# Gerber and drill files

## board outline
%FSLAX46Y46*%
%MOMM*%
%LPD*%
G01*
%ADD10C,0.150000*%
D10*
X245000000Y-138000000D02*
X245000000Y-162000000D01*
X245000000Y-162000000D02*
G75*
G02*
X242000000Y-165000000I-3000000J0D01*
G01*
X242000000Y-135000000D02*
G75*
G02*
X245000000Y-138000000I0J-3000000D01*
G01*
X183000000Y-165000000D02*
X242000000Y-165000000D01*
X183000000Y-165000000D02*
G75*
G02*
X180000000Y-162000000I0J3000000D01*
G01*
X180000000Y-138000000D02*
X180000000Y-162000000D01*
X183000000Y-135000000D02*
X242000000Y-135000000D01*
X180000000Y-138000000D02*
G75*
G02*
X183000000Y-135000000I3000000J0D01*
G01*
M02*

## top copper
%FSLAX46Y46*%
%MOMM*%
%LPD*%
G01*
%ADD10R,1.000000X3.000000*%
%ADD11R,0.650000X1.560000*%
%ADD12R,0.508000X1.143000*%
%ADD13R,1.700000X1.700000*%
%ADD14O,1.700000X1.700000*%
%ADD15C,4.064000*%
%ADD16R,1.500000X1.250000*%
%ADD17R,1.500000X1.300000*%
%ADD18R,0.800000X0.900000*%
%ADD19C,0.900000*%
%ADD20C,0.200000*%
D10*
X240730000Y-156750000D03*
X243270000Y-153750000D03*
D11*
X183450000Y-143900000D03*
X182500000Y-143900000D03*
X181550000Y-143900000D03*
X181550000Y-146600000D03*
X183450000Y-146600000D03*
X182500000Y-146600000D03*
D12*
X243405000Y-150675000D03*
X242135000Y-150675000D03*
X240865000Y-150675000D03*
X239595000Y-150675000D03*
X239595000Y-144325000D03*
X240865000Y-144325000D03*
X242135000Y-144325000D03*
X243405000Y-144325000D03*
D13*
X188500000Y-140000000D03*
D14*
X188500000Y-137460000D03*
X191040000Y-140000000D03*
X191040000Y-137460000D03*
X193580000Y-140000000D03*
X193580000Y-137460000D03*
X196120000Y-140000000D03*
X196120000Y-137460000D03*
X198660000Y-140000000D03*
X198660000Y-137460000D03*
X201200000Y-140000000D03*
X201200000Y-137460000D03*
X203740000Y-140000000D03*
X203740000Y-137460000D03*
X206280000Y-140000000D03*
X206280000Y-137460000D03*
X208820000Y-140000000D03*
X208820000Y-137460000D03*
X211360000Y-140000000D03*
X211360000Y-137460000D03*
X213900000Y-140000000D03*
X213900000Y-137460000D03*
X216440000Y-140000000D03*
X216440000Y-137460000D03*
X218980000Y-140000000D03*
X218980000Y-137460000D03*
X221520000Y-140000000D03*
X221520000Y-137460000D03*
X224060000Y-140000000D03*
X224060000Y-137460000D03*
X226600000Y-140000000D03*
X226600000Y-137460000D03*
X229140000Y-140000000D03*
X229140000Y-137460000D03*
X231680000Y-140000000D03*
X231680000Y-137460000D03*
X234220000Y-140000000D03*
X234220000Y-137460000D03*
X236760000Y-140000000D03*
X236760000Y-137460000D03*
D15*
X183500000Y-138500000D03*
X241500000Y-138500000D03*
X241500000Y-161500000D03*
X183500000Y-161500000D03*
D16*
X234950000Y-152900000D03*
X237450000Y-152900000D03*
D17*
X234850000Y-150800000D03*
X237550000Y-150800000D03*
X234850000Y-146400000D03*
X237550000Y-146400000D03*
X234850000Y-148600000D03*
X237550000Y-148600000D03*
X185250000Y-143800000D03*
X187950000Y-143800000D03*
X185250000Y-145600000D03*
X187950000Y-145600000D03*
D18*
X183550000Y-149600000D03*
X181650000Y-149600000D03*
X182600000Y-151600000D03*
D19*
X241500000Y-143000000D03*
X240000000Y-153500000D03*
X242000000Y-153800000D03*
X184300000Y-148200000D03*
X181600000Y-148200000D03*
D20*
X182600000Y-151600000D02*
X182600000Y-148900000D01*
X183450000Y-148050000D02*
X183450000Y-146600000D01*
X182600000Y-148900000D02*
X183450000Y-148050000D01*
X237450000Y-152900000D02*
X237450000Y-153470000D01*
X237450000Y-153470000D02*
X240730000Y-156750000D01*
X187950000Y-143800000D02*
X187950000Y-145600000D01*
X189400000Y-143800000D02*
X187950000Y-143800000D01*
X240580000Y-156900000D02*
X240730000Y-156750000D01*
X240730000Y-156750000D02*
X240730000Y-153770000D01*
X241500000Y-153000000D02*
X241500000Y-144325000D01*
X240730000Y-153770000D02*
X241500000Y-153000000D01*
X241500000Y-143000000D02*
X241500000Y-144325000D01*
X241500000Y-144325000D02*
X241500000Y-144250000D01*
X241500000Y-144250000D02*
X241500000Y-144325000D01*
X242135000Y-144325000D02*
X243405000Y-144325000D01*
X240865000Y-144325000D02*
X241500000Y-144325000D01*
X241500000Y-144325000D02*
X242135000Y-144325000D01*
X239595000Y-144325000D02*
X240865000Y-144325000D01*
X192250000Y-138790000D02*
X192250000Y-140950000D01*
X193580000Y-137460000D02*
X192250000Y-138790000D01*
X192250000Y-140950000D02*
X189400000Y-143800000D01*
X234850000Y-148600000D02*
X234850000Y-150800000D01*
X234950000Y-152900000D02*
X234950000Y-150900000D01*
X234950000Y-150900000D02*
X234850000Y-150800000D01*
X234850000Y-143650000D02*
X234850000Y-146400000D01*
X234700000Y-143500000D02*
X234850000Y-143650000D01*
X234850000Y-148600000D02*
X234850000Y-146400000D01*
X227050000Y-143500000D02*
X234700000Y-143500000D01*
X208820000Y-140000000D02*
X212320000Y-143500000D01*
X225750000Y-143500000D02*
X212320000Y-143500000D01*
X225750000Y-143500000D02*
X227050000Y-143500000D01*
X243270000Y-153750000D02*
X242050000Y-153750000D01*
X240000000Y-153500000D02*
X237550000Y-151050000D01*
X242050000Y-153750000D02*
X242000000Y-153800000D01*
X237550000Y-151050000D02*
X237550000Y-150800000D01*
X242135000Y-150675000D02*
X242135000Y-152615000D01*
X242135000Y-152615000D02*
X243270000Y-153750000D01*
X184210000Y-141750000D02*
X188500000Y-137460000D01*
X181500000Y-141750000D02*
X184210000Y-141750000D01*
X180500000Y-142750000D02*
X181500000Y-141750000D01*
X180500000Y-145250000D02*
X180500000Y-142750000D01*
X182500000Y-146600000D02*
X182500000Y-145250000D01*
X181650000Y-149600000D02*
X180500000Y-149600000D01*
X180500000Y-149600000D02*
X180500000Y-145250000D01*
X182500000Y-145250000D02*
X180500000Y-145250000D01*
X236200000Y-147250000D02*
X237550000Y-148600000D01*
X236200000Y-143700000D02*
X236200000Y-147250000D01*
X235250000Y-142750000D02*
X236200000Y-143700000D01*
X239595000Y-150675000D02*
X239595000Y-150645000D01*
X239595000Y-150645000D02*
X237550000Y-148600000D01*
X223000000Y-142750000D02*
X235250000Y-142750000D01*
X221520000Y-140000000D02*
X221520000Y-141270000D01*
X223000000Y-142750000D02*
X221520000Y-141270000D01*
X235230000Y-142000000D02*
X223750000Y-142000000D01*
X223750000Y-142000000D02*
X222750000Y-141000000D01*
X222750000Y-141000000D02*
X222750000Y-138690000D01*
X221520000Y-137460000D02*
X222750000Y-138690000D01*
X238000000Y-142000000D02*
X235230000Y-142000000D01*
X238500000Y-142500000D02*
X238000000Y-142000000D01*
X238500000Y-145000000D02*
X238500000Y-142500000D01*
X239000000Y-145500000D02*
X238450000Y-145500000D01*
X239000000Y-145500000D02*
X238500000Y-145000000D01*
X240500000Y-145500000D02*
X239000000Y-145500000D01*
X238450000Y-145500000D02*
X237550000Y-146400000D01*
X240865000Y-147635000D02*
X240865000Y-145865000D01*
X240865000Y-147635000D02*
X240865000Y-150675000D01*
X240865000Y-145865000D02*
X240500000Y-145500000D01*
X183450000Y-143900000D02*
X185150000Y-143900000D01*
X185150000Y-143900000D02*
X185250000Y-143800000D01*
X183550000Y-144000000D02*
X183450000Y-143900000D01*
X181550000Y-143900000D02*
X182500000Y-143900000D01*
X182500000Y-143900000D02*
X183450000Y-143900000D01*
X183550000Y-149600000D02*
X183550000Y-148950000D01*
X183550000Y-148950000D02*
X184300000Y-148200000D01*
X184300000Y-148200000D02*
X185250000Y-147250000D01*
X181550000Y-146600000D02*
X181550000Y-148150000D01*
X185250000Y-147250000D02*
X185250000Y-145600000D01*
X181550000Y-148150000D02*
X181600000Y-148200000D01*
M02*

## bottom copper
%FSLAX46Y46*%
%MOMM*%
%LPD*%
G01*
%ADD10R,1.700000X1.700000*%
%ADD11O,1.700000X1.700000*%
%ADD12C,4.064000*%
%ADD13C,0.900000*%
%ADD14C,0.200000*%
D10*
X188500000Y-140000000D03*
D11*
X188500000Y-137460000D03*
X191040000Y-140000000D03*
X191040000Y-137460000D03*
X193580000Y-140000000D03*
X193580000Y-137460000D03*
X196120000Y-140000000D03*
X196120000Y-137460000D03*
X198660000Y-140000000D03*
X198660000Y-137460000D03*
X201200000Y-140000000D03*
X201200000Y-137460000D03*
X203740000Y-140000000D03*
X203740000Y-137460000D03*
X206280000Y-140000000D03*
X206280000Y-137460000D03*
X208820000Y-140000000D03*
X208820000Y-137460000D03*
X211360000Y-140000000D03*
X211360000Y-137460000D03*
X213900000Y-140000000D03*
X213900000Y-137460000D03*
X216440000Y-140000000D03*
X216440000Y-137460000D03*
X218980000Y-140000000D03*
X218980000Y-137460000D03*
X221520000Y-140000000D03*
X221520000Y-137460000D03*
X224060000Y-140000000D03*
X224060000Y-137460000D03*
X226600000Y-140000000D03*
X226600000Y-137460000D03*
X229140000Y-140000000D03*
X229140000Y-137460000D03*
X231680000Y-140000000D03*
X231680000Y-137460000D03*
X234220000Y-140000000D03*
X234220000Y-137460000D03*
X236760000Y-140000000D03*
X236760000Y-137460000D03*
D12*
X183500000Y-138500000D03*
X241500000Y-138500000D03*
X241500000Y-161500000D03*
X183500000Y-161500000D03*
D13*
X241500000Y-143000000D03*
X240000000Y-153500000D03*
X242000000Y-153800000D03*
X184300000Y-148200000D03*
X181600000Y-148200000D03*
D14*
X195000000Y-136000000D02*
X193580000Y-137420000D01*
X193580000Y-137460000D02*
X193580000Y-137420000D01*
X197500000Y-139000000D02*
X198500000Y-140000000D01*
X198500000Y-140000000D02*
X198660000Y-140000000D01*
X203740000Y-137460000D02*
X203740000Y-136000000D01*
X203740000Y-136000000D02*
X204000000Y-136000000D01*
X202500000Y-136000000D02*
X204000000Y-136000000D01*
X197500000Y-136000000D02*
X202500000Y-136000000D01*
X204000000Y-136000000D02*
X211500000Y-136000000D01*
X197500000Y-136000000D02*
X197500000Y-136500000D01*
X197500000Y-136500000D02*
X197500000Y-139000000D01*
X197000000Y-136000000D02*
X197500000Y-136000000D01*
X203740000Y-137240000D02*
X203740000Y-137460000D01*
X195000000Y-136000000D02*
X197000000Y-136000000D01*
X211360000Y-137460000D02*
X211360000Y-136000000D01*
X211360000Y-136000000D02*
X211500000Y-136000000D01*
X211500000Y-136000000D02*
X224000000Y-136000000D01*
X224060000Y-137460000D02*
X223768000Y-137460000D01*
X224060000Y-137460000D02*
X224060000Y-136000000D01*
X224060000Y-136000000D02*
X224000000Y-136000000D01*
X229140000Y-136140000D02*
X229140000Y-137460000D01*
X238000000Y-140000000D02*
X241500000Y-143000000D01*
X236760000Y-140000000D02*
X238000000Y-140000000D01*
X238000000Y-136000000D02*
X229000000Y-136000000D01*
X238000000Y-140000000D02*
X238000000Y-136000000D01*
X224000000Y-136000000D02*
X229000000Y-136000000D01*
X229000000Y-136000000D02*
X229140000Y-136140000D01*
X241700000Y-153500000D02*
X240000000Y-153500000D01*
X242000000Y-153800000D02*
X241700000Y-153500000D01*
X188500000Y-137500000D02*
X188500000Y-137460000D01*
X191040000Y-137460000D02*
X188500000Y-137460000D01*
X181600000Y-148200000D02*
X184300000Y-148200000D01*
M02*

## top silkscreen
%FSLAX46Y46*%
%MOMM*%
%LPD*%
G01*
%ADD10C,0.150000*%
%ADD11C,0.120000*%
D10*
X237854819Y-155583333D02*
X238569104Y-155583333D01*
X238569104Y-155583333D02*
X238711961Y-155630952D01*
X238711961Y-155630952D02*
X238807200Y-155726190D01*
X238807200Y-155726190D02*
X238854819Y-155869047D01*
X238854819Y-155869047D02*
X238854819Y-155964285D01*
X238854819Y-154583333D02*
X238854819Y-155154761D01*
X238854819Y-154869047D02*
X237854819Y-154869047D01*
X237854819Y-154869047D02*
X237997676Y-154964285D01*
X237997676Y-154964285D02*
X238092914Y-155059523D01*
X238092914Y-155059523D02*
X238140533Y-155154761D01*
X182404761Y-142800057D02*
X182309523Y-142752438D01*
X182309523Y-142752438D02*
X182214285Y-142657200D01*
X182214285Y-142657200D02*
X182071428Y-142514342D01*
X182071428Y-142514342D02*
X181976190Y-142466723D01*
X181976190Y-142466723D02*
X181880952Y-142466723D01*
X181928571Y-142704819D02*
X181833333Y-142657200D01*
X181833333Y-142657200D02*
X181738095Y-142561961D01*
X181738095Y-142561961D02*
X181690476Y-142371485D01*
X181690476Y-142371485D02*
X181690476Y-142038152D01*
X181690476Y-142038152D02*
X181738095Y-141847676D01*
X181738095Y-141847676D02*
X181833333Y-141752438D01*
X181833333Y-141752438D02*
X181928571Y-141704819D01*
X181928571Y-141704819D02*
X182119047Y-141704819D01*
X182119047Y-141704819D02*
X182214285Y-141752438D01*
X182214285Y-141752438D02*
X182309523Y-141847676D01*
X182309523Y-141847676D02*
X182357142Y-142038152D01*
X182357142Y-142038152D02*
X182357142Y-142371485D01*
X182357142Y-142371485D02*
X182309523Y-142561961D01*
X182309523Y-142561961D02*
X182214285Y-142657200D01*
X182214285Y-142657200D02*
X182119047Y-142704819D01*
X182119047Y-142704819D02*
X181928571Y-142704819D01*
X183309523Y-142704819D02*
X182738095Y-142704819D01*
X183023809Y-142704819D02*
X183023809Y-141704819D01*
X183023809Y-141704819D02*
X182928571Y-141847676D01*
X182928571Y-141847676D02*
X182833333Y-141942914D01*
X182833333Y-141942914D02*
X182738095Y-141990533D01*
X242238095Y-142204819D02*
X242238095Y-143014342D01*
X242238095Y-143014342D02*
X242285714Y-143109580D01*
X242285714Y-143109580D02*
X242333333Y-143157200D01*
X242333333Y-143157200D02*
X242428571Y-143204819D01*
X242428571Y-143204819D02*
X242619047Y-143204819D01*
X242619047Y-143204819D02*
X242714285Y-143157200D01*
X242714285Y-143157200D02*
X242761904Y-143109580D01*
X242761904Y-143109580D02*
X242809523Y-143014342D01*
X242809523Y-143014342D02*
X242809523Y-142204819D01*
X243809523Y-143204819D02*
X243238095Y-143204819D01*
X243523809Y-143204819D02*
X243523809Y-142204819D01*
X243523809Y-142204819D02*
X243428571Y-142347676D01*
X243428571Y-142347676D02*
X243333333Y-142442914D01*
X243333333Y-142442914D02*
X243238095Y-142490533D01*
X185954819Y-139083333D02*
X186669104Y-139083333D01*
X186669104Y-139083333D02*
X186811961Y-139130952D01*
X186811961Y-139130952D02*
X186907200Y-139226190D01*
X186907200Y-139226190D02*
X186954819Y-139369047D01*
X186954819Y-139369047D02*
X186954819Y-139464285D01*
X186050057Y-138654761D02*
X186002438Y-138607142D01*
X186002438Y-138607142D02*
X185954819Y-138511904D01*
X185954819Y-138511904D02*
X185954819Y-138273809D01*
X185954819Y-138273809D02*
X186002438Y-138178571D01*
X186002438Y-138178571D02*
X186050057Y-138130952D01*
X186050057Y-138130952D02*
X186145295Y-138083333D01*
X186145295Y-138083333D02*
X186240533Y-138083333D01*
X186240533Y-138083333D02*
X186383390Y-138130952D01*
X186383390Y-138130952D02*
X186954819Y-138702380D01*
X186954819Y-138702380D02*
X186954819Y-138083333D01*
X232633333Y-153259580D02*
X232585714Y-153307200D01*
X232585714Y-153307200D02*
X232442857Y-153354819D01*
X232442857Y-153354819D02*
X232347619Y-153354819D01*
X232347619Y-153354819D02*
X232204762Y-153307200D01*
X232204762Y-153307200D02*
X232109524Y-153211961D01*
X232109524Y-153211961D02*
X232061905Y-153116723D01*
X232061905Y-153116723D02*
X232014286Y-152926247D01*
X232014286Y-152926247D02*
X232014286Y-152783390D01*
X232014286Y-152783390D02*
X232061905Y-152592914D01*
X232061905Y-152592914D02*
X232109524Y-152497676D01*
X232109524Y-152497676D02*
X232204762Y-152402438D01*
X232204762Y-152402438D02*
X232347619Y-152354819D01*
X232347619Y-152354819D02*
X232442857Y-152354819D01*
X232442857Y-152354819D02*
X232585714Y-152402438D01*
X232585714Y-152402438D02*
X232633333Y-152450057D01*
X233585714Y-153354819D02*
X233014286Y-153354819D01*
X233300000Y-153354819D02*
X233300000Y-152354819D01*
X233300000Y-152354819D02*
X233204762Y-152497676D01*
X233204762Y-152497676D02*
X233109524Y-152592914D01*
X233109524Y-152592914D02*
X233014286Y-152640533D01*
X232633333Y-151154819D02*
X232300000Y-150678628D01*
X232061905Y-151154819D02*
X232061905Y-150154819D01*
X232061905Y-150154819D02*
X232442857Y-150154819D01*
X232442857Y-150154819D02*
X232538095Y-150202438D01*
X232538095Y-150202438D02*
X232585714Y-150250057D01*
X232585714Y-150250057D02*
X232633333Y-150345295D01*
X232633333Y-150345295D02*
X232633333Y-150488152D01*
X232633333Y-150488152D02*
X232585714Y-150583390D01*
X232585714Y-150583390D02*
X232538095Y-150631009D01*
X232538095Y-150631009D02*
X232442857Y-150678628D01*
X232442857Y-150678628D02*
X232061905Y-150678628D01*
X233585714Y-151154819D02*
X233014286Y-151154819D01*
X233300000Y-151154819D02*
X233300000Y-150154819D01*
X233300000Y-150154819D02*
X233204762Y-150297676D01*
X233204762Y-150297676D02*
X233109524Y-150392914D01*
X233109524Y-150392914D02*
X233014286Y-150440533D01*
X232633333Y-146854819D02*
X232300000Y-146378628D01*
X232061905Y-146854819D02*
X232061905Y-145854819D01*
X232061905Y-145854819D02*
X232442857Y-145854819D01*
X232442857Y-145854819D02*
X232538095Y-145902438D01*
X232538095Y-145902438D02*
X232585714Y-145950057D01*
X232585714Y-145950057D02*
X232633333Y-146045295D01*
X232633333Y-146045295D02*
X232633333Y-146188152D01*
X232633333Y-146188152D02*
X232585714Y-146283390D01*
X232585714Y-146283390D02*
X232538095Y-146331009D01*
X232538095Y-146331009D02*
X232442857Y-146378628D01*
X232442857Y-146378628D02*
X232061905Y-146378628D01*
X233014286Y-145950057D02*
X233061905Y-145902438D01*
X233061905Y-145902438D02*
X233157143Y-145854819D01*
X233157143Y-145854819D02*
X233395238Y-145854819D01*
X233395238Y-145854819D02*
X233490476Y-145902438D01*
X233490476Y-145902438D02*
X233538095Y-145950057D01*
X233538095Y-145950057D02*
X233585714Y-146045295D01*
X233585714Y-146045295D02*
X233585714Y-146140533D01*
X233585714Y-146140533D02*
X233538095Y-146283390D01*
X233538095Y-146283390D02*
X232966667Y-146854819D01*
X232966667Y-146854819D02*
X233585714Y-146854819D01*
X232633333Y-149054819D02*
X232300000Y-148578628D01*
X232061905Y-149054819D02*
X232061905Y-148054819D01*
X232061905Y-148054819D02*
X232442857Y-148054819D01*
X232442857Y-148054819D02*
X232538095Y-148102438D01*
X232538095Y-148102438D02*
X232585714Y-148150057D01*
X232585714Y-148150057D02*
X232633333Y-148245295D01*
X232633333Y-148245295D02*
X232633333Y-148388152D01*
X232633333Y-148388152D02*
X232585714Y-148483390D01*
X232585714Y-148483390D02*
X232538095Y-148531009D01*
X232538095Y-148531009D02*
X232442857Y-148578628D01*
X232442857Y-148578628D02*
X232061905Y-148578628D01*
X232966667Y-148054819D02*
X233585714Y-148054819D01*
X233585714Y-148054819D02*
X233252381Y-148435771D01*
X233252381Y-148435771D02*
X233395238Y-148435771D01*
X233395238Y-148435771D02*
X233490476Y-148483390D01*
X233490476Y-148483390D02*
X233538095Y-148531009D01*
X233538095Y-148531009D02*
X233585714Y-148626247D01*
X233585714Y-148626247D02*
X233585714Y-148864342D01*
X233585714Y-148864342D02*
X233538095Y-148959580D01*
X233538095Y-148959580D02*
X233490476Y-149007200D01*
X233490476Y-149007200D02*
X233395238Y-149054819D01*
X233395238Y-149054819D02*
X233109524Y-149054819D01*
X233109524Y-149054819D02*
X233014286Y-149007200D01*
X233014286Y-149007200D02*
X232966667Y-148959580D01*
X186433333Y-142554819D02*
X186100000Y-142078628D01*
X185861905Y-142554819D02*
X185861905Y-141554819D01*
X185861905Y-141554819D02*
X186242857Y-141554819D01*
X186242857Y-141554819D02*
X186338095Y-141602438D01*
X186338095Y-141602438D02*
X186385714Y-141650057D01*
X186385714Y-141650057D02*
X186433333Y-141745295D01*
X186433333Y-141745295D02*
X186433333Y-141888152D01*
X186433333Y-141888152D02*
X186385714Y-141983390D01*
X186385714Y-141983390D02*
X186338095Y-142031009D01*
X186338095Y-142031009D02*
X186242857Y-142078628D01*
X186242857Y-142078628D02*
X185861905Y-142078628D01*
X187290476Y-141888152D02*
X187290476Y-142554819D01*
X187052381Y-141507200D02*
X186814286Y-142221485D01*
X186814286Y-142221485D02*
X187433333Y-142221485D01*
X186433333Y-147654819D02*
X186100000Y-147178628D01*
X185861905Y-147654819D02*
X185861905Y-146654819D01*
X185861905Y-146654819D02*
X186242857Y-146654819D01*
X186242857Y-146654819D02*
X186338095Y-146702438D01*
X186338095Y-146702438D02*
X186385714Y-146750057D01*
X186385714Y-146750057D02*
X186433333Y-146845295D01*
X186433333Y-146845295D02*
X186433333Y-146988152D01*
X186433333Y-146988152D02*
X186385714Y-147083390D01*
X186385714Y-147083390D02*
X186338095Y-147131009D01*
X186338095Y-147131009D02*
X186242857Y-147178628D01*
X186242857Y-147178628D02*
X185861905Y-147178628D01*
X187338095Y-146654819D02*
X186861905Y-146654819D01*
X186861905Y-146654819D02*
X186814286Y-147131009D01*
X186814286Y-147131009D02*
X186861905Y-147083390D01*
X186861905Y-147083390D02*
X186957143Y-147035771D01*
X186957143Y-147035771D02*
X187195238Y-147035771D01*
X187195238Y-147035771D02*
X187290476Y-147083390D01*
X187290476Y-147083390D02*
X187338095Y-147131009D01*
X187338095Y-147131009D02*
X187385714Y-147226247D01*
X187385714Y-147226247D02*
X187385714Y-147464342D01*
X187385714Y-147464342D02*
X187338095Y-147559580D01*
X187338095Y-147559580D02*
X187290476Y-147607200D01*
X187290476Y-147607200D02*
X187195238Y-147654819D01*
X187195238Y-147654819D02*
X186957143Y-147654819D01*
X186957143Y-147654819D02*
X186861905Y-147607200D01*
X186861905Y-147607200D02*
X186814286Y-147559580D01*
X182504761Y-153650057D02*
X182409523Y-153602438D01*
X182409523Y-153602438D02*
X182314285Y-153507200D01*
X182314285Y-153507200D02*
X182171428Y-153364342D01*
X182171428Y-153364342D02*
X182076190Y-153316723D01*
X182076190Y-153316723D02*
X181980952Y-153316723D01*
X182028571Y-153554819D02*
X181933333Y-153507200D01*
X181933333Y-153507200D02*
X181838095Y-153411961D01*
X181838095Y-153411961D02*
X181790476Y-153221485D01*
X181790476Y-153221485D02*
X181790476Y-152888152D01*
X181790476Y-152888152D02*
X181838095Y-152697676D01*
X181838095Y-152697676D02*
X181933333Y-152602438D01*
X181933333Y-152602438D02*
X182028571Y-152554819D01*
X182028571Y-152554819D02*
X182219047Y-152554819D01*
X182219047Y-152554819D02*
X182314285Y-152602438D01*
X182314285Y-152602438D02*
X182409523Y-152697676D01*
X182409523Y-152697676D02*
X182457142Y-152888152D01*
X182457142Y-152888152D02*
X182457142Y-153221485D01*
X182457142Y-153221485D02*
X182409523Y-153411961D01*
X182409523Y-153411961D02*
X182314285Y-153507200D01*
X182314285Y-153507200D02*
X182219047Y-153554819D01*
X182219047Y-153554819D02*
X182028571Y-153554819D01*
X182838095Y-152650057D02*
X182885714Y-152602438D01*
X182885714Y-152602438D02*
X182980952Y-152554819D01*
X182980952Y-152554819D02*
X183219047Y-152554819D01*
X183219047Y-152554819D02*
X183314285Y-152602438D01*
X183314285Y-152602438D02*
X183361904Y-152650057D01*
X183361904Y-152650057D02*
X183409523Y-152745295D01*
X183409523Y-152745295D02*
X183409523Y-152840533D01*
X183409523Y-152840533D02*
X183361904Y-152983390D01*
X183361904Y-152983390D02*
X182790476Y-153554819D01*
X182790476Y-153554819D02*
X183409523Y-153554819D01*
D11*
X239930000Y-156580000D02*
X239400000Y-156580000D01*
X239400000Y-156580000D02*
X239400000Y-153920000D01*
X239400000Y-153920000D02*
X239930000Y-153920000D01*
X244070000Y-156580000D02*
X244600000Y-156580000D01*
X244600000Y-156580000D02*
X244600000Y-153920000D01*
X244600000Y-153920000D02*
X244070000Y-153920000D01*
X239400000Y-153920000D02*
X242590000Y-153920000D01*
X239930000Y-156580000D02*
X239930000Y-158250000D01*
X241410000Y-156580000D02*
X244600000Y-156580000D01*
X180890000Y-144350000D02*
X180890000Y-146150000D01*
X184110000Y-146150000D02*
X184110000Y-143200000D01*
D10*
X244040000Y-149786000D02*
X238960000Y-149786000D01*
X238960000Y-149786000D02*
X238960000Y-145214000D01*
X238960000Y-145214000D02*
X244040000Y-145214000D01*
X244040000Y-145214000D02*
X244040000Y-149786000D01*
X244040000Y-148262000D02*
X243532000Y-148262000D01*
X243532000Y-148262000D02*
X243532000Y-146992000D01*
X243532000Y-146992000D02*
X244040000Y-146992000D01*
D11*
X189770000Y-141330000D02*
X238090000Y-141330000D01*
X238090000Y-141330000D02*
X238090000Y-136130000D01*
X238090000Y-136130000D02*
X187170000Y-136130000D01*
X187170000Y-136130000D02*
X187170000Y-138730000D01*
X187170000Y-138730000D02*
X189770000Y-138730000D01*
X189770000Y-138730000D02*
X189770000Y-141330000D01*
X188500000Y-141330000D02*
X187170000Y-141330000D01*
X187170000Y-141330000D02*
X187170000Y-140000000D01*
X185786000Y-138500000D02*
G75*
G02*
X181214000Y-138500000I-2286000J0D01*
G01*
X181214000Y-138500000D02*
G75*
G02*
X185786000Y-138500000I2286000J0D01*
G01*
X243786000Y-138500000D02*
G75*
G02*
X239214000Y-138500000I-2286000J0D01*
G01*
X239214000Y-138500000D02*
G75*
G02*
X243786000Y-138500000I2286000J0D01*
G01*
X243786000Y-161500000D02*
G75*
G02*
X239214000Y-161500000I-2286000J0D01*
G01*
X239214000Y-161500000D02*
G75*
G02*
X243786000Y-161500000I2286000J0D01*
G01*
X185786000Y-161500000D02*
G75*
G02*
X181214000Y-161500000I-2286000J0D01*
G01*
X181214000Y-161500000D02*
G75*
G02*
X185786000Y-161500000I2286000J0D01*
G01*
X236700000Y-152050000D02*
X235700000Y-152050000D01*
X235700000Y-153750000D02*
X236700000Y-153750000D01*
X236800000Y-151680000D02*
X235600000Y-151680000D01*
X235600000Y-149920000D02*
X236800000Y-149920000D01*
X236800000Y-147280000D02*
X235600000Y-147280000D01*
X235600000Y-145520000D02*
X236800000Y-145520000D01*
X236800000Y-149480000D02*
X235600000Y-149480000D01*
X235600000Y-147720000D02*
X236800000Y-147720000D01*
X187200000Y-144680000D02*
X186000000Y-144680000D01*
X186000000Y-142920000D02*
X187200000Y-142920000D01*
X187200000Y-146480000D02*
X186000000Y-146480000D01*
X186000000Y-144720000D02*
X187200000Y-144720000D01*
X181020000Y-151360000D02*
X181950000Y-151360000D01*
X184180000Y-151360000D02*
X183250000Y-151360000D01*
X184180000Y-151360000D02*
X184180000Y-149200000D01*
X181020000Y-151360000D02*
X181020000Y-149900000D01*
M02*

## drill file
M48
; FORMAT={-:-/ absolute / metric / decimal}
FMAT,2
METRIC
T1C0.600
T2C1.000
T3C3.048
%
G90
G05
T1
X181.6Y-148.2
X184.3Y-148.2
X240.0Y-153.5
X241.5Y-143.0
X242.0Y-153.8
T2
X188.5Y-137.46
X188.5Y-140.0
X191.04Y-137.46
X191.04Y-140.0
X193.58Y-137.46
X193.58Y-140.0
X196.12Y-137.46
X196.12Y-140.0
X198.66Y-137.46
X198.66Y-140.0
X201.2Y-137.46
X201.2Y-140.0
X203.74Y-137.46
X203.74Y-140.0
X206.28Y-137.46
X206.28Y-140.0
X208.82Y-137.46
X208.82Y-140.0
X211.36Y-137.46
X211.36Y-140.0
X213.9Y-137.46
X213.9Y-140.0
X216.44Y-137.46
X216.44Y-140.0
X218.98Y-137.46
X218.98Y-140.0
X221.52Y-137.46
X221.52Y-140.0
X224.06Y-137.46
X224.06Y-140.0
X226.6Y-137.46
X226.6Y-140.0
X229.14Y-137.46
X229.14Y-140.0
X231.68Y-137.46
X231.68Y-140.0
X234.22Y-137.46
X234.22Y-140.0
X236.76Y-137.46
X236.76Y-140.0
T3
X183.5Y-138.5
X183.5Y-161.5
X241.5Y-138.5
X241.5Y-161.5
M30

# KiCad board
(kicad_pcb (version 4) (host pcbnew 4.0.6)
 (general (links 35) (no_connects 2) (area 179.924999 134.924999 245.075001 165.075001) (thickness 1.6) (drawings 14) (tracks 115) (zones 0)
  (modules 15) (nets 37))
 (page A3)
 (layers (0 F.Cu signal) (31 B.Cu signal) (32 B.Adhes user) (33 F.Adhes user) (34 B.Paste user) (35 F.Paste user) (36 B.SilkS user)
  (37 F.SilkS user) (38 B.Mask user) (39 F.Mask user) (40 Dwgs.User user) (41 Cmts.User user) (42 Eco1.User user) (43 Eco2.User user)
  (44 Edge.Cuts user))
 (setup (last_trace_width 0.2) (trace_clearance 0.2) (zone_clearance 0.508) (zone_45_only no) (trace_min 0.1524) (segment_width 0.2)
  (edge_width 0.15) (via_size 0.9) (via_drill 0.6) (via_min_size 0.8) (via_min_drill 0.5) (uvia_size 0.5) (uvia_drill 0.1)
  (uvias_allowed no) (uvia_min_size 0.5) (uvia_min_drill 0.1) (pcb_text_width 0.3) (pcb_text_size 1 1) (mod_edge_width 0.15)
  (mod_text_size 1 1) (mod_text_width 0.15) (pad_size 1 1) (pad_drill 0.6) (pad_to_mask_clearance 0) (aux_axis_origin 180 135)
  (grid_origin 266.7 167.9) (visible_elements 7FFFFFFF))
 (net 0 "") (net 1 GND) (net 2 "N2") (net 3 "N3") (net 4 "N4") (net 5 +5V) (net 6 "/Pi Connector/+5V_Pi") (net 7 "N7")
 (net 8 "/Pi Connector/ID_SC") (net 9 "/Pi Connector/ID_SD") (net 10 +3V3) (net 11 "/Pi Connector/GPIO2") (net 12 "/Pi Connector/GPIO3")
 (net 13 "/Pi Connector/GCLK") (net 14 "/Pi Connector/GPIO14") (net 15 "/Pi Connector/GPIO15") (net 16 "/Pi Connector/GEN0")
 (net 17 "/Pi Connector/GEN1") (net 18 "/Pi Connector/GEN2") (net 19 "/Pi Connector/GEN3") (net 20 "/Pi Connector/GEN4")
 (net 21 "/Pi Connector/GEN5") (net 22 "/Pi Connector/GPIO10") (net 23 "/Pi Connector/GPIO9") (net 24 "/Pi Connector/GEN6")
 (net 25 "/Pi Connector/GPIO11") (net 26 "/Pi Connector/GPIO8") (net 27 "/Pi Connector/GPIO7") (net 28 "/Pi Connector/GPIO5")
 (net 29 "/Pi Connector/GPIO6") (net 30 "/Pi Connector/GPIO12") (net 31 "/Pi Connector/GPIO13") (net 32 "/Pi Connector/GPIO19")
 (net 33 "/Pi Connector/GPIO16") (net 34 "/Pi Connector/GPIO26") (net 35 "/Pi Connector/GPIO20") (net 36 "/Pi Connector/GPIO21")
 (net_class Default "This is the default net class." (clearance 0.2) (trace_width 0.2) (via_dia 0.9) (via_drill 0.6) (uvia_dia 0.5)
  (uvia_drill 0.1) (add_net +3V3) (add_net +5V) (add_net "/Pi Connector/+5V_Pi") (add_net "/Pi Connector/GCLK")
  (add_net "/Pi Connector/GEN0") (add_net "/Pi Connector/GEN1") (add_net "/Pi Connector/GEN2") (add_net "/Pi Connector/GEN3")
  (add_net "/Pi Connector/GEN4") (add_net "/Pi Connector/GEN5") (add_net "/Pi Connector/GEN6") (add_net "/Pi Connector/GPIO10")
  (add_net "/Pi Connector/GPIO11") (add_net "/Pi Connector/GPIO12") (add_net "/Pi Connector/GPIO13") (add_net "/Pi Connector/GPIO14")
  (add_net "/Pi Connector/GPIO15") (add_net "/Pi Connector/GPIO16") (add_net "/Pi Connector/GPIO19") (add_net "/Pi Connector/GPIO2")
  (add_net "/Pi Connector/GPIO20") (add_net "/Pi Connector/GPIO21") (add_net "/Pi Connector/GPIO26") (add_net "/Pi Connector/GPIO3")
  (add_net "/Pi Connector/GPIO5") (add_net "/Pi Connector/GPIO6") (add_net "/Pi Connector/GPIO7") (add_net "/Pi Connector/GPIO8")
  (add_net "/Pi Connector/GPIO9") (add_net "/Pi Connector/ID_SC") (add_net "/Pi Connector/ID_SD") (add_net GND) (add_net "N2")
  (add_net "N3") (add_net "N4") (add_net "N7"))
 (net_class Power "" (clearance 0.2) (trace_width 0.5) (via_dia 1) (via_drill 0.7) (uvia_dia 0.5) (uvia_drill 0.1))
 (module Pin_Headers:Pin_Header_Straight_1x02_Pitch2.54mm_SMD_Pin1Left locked (layer F.Cu) (at 242 155.25 90)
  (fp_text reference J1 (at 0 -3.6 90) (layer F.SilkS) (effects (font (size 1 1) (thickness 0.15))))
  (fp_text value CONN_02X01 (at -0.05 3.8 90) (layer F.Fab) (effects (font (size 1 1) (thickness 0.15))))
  (fp_line (start -1.33 -2.07) (end -1.33 -2.6) (layer F.SilkS) (width 0.12))
  (fp_line (start -1.33 -2.6) (end 1.33 -2.6) (layer F.SilkS) (width 0.12))
  (fp_line (start 1.33 -2.6) (end 1.33 -2.07) (layer F.SilkS) (width 0.12))
  (fp_line (start -1.33 2.07) (end -1.33 2.6) (layer F.SilkS) (width 0.12))
  (fp_line (start -1.33 2.6) (end 1.33 2.6) (layer F.SilkS) (width 0.12))
  (fp_line (start 1.33 2.6) (end 1.33 2.07) (layer F.SilkS) (width 0.12))
  (fp_line (start 1.33 -2.6) (end 1.33 0.59) (layer F.SilkS) (width 0.12))
  (fp_line (start -1.33 -2.07) (end -3 -2.07) (layer F.SilkS) (width 0.12))
  (fp_line (start -1.33 -0.59) (end -1.33 2.6) (layer F.SilkS) (width 0.12))
  (pad 1 smd rect (at -1.5 -1.27 90) (size 3 1) (layers F.Cu F.Paste F.Mask) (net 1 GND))
  (pad 2 smd rect (at 1.5 1.27 90) (size 3 1) (layers F.Cu F.Paste F.Mask) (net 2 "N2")))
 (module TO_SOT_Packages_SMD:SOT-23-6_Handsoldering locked (layer F.Cu) (at 182.5 145.25 270)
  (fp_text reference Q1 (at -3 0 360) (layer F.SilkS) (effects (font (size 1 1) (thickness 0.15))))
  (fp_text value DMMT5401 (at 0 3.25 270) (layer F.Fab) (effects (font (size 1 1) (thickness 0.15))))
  (fp_line (start -0.9 1.61) (end 0.9 1.61) (layer F.SilkS) (width 0.12))
  (fp_line (start 0.9 -1.61) (end -2.05 -1.61) (layer F.SilkS) (width 0.12))
  (pad 1 smd rect (at -1.35 -0.95 270) (size 1.56 0.65) (layers F.Cu F.Paste F.Mask) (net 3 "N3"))
  (pad 2 smd rect (at -1.35 0 270) (size 1.56 0.65) (layers F.Cu F.Paste F.Mask) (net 3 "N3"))
  (pad 3 smd rect (at -1.35 0.95 270) (size 1.56 0.65) (layers F.Cu F.Paste F.Mask) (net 3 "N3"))
  (pad 4 smd rect (at 1.35 0.95 270) (size 1.56 0.65) (layers F.Cu F.Paste F.Mask) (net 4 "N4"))
  (pad 6 smd rect (at 1.35 -0.95 270) (size 1.56 0.65) (layers F.Cu F.Paste F.Mask) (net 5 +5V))
  (pad 5 smd rect (at 1.35 0 270) (size 1.56 0.65) (layers F.Cu F.Paste F.Mask) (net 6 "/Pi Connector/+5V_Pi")))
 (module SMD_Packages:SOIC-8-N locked (layer F.Cu) (at 241.5 147.5 180)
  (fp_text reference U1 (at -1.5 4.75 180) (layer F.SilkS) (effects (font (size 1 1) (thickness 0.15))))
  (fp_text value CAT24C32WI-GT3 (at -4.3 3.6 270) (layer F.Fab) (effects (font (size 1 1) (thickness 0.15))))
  (fp_line (start -2.54 -2.286) (end 2.54 -2.286) (layer F.SilkS) (width 0.15))
  (fp_line (start 2.54 -2.286) (end 2.54 2.286) (layer F.SilkS) (width 0.15))
  (fp_line (start 2.54 2.286) (end -2.54 2.286) (layer F.SilkS) (width 0.15))
  (fp_line (start -2.54 2.286) (end -2.54 -2.286) (layer F.SilkS) (width 0.15))
  (fp_line (start -2.54 -0.762) (end -2.032 -0.762) (layer F.SilkS) (width 0.15))
  (fp_line (start -2.032 -0.762) (end -2.032 0.508) (layer F.SilkS) (width 0.15))
  (fp_line (start -2.032 0.508) (end -2.54 0.508) (layer F.SilkS) (width 0.15))
  (pad 8 smd rect (at -1.905 -3.175 180) (size 0.508 1.143) (layers F.Cu F.Paste F.Mask) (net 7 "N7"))
  (pad 7 smd rect (at -0.635 -3.175 180) (size 0.508 1.143) (layers F.Cu F.Paste F.Mask) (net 2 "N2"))
  (pad 6 smd rect (at 0.635 -3.175 180) (size 0.508 1.143) (layers F.Cu F.Paste F.Mask) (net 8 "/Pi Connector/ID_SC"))
  (pad 5 smd rect (at 1.905 -3.175 180) (size 0.508 1.143) (layers F.Cu F.Paste F.Mask) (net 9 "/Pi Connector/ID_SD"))
  (pad 4 smd rect (at 1.905 3.175 180) (size 0.508 1.143) (layers F.Cu F.Paste F.Mask) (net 1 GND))
  (pad 3 smd rect (at 0.635 3.175 180) (size 0.508 1.143) (layers F.Cu F.Paste F.Mask) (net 1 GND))
  (pad 2 smd rect (at -0.635 3.175 180) (size 0.508 1.143) (layers F.Cu F.Paste F.Mask) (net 1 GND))
  (pad 1 smd rect (at -1.905 3.175 180) (size 0.508 1.143) (layers F.Cu F.Paste F.Mask) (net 1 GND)))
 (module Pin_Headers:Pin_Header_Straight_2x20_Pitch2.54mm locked (layer F.Cu) (at 188.5 140 90)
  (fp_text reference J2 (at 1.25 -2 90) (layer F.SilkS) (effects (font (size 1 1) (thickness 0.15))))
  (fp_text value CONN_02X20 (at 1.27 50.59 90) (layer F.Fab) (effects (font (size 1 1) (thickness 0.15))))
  (fp_line (start -1.33 1.27) (end -1.33 49.59) (layer F.SilkS) (width 0.12))
  (fp_line (start -1.33 49.59) (end 3.87 49.59) (layer F.SilkS) (width 0.12))
  (fp_line (start 3.87 49.59) (end 3.87 -1.33) (layer F.SilkS) (width 0.12))
  (fp_line (start 3.87 -1.33) (end 1.27 -1.33) (layer F.SilkS) (width 0.12))
  (fp_line (start 1.27 -1.33) (end 1.27 1.27) (layer F.SilkS) (width 0.12))
  (fp_line (start 1.27 1.27) (end -1.33 1.27) (layer F.SilkS) (width 0.12))
  (fp_line (start -1.33 0) (end -1.33 -1.33) (layer F.SilkS) (width 0.12))
  (fp_line (start -1.33 -1.33) (end 0 -1.33) (layer F.SilkS) (width 0.12))
  (pad 1 thru_hole rect (at 0 0 90) (size 1.7 1.7) (drill 1) (layers *.Cu *.Mask) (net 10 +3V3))
  (pad 2 thru_hole oval (at 2.54 0 90) (size 1.7 1.7) (drill 1) (layers *.Cu *.Mask) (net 6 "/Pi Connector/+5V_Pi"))
  (pad 3 thru_hole oval (at 0 2.54 90) (size 1.7 1.7) (drill 1) (layers *.Cu *.Mask) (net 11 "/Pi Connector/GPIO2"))
  (pad 4 thru_hole oval (at 2.54 2.54 90) (size 1.7 1.7) (drill 1) (layers *.Cu *.Mask) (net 6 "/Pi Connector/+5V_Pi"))
  (pad 5 thru_hole oval (at 0 5.08 90) (size 1.7 1.7) (drill 1) (layers *.Cu *.Mask) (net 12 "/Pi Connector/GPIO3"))
  (pad 6 thru_hole oval (at 2.54 5.08 90) (size 1.7 1.7) (drill 1) (layers *.Cu *.Mask) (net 1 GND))
  (pad 7 thru_hole oval (at 0 7.62 90) (size 1.7 1.7) (drill 1) (layers *.Cu *.Mask) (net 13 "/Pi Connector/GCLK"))
  (pad 8 thru_hole oval (at 2.54 7.62 90) (size 1.7 1.7) (drill 1) (layers *.Cu *.Mask) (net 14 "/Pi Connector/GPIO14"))
  (pad 9 thru_hole oval (at 0 10.16 90) (size 1.7 1.7) (drill 1) (layers *.Cu *.Mask) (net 1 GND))
  (pad 10 thru_hole oval (at 2.54 10.16 90) (size 1.7 1.7) (drill 1) (layers *.Cu *.Mask) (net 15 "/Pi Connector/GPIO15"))
  (pad 11 thru_hole oval (at 0 12.7 90) (size 1.7 1.7) (drill 1) (layers *.Cu *.Mask) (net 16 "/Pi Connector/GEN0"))
  (pad 12 thru_hole oval (at 2.54 12.7 90) (size 1.7 1.7) (drill 1) (layers *.Cu *.Mask) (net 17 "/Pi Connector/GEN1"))
  (pad 13 thru_hole oval (at 0 15.24 90) (size 1.7 1.7) (drill 1) (layers *.Cu *.Mask) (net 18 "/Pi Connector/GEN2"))
  (pad 14 thru_hole oval (at 2.54 15.24 90) (size 1.7 1.7) (drill 1) (layers *.Cu *.Mask) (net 1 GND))
  (pad 15 thru_hole oval (at 0 17.78 90) (size 1.7 1.7) (drill 1) (layers *.Cu *.Mask) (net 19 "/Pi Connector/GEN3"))
  (pad 16 thru_hole oval (at 2.54 17.78 90) (size 1.7 1.7) (drill 1) (layers *.Cu *.Mask) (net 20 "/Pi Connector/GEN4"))
  (pad 17 thru_hole oval (at 0 20.32 90) (size 1.7 1.7) (drill 1) (layers *.Cu *.Mask) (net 10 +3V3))
  (pad 18 thru_hole oval (at 2.54 20.32 90) (size 1.7 1.7) (drill 1) (layers *.Cu *.Mask) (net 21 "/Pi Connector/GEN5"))
  (pad 19 thru_hole oval (at 0 22.86 90) (size 1.7 1.7) (drill 1) (layers *.Cu *.Mask) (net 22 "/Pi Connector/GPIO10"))
  (pad 20 thru_hole oval (at 2.54 22.86 90) (size 1.7 1.7) (drill 1) (layers *.Cu *.Mask) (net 1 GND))
  (pad 21 thru_hole oval (at 0 25.4 90) (size 1.7 1.7) (drill 1) (layers *.Cu *.Mask) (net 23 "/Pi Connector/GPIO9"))
  (pad 22 thru_hole oval (at 2.54 25.4 90) (size 1.7 1.7) (drill 1) (layers *.Cu *.Mask) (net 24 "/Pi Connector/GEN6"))
  (pad 23 thru_hole oval (at 0 27.94 90) (size 1.7 1.7) (drill 1) (layers *.Cu *.Mask) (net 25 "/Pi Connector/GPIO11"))
  (pad 24 thru_hole oval (at 2.54 27.94 90) (size 1.7 1.7) (drill 1) (layers *.Cu *.Mask) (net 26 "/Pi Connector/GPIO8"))
  (pad 25 thru_hole oval (at 0 30.48 90) (size 1.7 1.7) (drill 1) (layers *.Cu *.Mask) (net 1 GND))
  (pad 26 thru_hole oval (at 2.54 30.48 90) (size 1.7 1.7) (drill 1) (layers *.Cu *.Mask) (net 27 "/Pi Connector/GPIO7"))
  (pad 27 thru_hole oval (at 0 33.02 90) (size 1.7 1.7) (drill 1) (layers *.Cu *.Mask) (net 9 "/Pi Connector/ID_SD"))
  (pad 28 thru_hole oval (at 2.54 33.02 90) (size 1.7 1.7) (drill 1) (layers *.Cu *.Mask) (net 8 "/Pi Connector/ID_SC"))
  (pad 29 thru_hole oval (at 0 35.56 90) (size 1.7 1.7) (drill 1) (layers *.Cu *.Mask) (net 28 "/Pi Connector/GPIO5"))
  (pad 30 thru_hole oval (at 2.54 35.56 90) (size 1.7 1.7) (drill 1) (layers *.Cu *.Mask) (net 1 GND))
  (pad 31 thru_hole oval (at 0 38.1 90) (size 1.7 1.7) (drill 1) (layers *.Cu *.Mask) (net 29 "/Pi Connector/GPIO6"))
  (pad 32 thru_hole oval (at 2.54 38.1 90) (size 1.7 1.7) (drill 1) (layers *.Cu *.Mask) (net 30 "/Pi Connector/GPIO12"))
  (pad 33 thru_hole oval (at 0 40.64 90) (size 1.7 1.7) (drill 1) (layers *.Cu *.Mask) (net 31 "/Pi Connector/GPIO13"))
  (pad 34 thru_hole oval (at 2.54 40.64 90) (size 1.7 1.7) (drill 1) (layers *.Cu *.Mask) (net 1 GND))
  (pad 35 thru_hole oval (at 0 43.18 90) (size 1.7 1.7) (drill 1) (layers *.Cu *.Mask) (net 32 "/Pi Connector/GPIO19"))
  (pad 36 thru_hole oval (at 2.54 43.18 90) (size 1.7 1.7) (drill 1) (layers *.Cu *.Mask) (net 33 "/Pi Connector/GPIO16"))
  (pad 37 thru_hole oval (at 0 45.72 90) (size 1.7 1.7) (drill 1) (layers *.Cu *.Mask) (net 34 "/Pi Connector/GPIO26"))
  (pad 38 thru_hole oval (at 2.54 45.72 90) (size 1.7 1.7) (drill 1) (layers *.Cu *.Mask) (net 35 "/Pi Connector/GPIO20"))
  (pad 39 thru_hole oval (at 0 48.26 90) (size 1.7 1.7) (drill 1) (layers *.Cu *.Mask) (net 1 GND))
  (pad 40 thru_hole oval (at 2.54 48.26 90) (size 1.7 1.7) (drill 1) (layers *.Cu *.Mask) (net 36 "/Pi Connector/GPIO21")))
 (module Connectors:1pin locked (layer F.Cu) (at 183.5 138.5)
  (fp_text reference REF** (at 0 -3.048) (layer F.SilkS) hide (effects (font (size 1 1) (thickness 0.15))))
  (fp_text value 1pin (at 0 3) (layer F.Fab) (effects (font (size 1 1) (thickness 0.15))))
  (fp_circle (center 0 0) (end 0 -2.286) (layer F.SilkS) (width 0.12))
  (pad 1 thru_hole circle (at 0 0) (size 4.064 4.064) (drill 3.048) (layers *.Cu *.Mask)))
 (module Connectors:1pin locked (layer F.Cu) (at 241.5 138.5)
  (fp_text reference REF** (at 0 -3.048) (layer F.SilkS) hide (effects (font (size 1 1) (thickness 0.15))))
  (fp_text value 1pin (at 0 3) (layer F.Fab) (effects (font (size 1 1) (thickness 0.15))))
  (fp_circle (center 0 0) (end 0 -2.286) (layer F.SilkS) (width 0.12))
  (pad 1 thru_hole circle (at 0 0) (size 4.064 4.064) (drill 3.048) (layers *.Cu *.Mask)))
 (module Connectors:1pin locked (layer F.Cu) (at 241.5 161.5)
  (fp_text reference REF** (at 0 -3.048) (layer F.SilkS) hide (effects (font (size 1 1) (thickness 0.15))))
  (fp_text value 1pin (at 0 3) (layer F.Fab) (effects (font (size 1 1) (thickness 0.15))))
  (fp_circle (center 0 0) (end 0 -2.286) (layer F.SilkS) (width 0.12))
  (pad 1 thru_hole circle (at 0 0) (size 4.064 4.064) (drill 3.048) (layers *.Cu *.Mask)))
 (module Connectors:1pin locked (layer F.Cu) (at 183.5 161.5)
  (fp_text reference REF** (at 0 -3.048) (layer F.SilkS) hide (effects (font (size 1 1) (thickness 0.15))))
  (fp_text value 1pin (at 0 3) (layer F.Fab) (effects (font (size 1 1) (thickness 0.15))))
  (fp_circle (center 0 0) (end 0 -2.286) (layer F.SilkS) (width 0.12))
  (pad 1 thru_hole circle (at 0 0) (size 4.064 4.064) (drill 3.048) (layers *.Cu *.Mask)))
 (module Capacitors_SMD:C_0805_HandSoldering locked (layer F.Cu) (at 236.2 152.9)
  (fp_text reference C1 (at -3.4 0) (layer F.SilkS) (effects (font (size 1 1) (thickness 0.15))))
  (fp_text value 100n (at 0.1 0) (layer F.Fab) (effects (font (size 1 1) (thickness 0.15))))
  (fp_line (start 0.5 -0.85) (end -0.5 -0.85) (layer F.SilkS) (width 0.12))
  (fp_line (start -0.5 0.85) (end 0.5 0.85) (layer F.SilkS) (width 0.12))
  (pad 1 smd rect (at -1.25 0) (size 1.5 1.25) (layers F.Cu F.Paste F.Mask) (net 10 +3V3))
  (pad 2 smd rect (at 1.25 0) (size 1.5 1.25) (layers F.Cu F.Paste F.Mask) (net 1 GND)))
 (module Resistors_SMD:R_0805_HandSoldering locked (layer F.Cu) (at 236.2 150.8)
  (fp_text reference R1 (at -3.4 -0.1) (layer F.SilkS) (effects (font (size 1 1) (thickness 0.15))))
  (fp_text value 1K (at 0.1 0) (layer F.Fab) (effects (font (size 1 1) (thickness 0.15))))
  (fp_line (start 0.6 0.88) (end -0.6 0.88) (layer F.SilkS) (width 0.12))
  (fp_line (start -0.6 -0.88) (end 0.6 -0.88) (layer F.SilkS) (width 0.12))
  (pad 1 smd rect (at -1.35 0) (size 1.5 1.3) (layers F.Cu F.Paste F.Mask) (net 10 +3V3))
  (pad 2 smd rect (at 1.35 0) (size 1.5 1.3) (layers F.Cu F.Paste F.Mask) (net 2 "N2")))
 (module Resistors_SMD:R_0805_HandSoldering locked (layer F.Cu) (at 236.2 146.4)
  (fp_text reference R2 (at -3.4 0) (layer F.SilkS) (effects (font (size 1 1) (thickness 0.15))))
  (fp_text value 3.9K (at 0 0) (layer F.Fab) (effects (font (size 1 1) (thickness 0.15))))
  (fp_line (start 0.6 0.88) (end -0.6 0.88) (layer F.SilkS) (width 0.12))
  (fp_line (start -0.6 -0.88) (end 0.6 -0.88) (layer F.SilkS) (width 0.12))
  (pad 1 smd rect (at -1.35 0) (size 1.5 1.3) (layers F.Cu F.Paste F.Mask) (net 10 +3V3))
  (pad 2 smd rect (at 1.35 0) (size 1.5 1.3) (layers F.Cu F.Paste F.Mask) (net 8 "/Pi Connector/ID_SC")))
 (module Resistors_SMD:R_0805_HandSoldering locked (layer F.Cu) (at 236.2 148.6)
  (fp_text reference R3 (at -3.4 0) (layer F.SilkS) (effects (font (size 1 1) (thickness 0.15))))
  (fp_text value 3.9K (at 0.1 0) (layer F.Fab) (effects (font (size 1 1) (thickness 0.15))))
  (fp_line (start 0.6 0.88) (end -0.6 0.88) (layer F.SilkS) (width 0.12))
  (fp_line (start -0.6 -0.88) (end 0.6 -0.88) (layer F.SilkS) (width 0.12))
  (pad 1 smd rect (at -1.35 0) (size 1.5 1.3) (layers F.Cu F.Paste F.Mask) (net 10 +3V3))
  (pad 2 smd rect (at 1.35 0) (size 1.5 1.3) (layers F.Cu F.Paste F.Mask) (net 9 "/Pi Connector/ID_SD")))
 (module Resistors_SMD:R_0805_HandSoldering (layer F.Cu) (at 186.6 143.8)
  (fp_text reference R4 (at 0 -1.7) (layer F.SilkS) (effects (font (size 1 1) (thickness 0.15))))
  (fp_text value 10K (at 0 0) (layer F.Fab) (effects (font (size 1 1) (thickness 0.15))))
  (fp_line (start 0.6 0.88) (end -0.6 0.88) (layer F.SilkS) (width 0.12))
  (fp_line (start -0.6 -0.88) (end 0.6 -0.88) (layer F.SilkS) (width 0.12))
  (pad 1 smd rect (at -1.35 0) (size 1.5 1.3) (layers F.Cu F.Paste F.Mask) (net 3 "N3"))
  (pad 2 smd rect (at 1.35 0) (size 1.5 1.3) (layers F.Cu F.Paste F.Mask) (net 1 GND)))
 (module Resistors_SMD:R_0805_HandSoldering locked (layer F.Cu) (at 186.6 145.6)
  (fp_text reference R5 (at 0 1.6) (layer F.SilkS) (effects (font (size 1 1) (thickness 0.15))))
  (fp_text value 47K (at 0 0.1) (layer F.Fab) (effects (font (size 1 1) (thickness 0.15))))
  (fp_line (start 0.6 0.88) (end -0.6 0.88) (layer F.SilkS) (width 0.12))
  (fp_line (start -0.6 -0.88) (end 0.6 -0.88) (layer F.SilkS) (width 0.12))
  (pad 1 smd rect (at -1.35 0) (size 1.5 1.3) (layers F.Cu F.Paste F.Mask) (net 4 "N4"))
  (pad 2 smd rect (at 1.35 0) (size 1.5 1.3) (layers F.Cu F.Paste F.Mask) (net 1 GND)))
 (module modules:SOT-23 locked (layer F.Cu) (at 182.6 150.6 180)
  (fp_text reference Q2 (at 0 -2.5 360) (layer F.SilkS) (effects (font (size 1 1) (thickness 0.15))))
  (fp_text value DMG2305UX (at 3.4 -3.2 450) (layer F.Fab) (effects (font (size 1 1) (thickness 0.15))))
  (fp_line (start 1.58 -0.76) (end 0.65 -0.76) (layer F.SilkS) (width 0.12))
  (fp_line (start -1.58 -0.76) (end -0.65 -0.76) (layer F.SilkS) (width 0.12))
  (fp_line (start -1.58 -0.76) (end -1.58 1.4) (layer F.SilkS) (width 0.12))
  (fp_line (start 1.58 -0.76) (end 1.58 0.7) (layer F.SilkS) (width 0.12))
  (pad 1 smd rect (at -0.95 1 270) (size 0.9 0.8) (layers F.Cu F.Paste F.Mask) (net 4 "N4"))
  (pad 2 smd rect (at 0.95 1 270) (size 0.9 0.8) (layers F.Cu F.Paste F.Mask) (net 6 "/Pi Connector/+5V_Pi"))
  (pad 3 smd rect (at 0 -1 270) (size 0.9 0.8) (layers F.Cu F.Paste F.Mask) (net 5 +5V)))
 (gr_line (start 245 138) (end 245 162) (angle 90) (layer Edge.Cuts) (width 0.15))
 (gr_arc (start 242 162) (end 245 162) (angle 90) (layer Edge.Cuts) (width 0.15))
 (gr_arc (start 242 138) (end 242 135) (angle 90) (layer Edge.Cuts) (width 0.15))
 (gr_line (start 183 165) (end 242 165) (angle 90) (layer Edge.Cuts) (width 0.15))
 (gr_arc (start 183 162) (end 183 165) (angle 90) (layer Edge.Cuts) (width 0.15))
 (gr_line (start 180 138) (end 180 162) (angle 90) (layer Edge.Cuts) (width 0.15))
 (gr_line (start 183 135) (end 242 135) (angle 90) (layer Edge.Cuts) (width 0.15))
 (gr_arc (start 183 138) (end 180 138) (angle 90) (layer Edge.Cuts) (width 0.15))
 (segment (start 182.6 151.6) (end 182.6 148.9) (width 0.2) (layer F.Cu) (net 5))
 (segment (start 183.45 148.05) (end 183.45 146.6) (width 0.2) (layer F.Cu) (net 5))
 (segment (start 182.6 148.9) (end 183.45 148.05) (width 0.2) (layer F.Cu) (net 5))
 (segment (start 237.45 152.9) (end 237.45 153.47) (width 0.2) (layer F.Cu) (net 1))
 (segment (start 237.45 153.47) (end 240.73 156.75) (width 0.2) (layer F.Cu) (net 1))
 (segment (start 187.95 143.8) (end 187.95 145.6) (width 0.2) (layer F.Cu) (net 1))
 (segment (start 189.4 143.8) (end 187.95 143.8) (width 0.2) (layer F.Cu) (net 1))
 (segment (start 240.58 156.9) (end 240.73 156.75) (width 0.2) (layer F.Cu) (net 1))
 (segment (start 240.73 156.75) (end 240.73 153.77) (width 0.2) (layer F.Cu) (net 1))
 (segment (start 241.5 153) (end 241.5 144.325) (width 0.2) (layer F.Cu) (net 1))
 (segment (start 240.73 153.77) (end 241.5 153) (width 0.2) (layer F.Cu) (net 1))
 (segment (start 241.5 143) (end 241.5 144.325) (width 0.2) (layer F.Cu) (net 1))
 (segment (start 241.5 144.325) (end 241.5 144.25) (width 0.2) (layer F.Cu) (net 1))
 (segment (start 241.5 144.25) (end 241.5 144.325) (width 0.2) (layer F.Cu) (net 1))
 (segment (start 242.135 144.325) (end 243.405 144.325) (width 0.2) (layer F.Cu) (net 1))
 (segment (start 240.865 144.325) (end 241.5 144.325) (width 0.2) (layer F.Cu) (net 1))
 (segment (start 241.5 144.325) (end 242.135 144.325) (width 0.2) (layer F.Cu) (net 1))
 (segment (start 239.595 144.325) (end 240.865 144.325) (width 0.2) (layer F.Cu) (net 1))
 (segment (start 192.25 138.79) (end 192.25 140.95) (width 0.2) (layer F.Cu) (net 1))
 (segment (start 193.58 137.46) (end 192.25 138.79) (width 0.2) (layer F.Cu) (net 1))
 (segment (start 192.25 140.95) (end 189.4 143.8) (width 0.2) (layer F.Cu) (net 1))
 (segment (start 195 136) (end 193.58 137.42) (width 0.2) (layer B.Cu) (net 1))
 (segment (start 193.58 137.46) (end 193.58 137.42) (width 0.2) (layer B.Cu) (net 1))
 (segment (start 197.5 139) (end 198.5 140) (width 0.2) (layer B.Cu) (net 1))
 (segment (start 198.5 140) (end 198.66 140) (width 0.2) (layer B.Cu) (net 1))
 (segment (start 203.74 137.46) (end 203.74 136) (width 0.2) (layer B.Cu) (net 1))
 (segment (start 203.74 136) (end 204 136) (width 0.2) (layer B.Cu) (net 1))
 (segment (start 202.5 136) (end 204 136) (width 0.2) (layer B.Cu) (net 1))
 (segment (start 197.5 136) (end 202.5 136) (width 0.2) (layer B.Cu) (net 1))
 (segment (start 204 136) (end 211.5 136) (width 0.2) (layer B.Cu) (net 1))
 (segment (start 197.5 136) (end 197.5 136.5) (width 0.2) (layer B.Cu) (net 1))
 (segment (start 197.5 136.5) (end 197.5 139) (width 0.2) (layer B.Cu) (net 1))
 (segment (start 197 136) (end 197.5 136) (width 0.2) (layer B.Cu) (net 1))
 (segment (start 203.74 137.24) (end 203.74 137.46) (width 0.2) (layer B.Cu) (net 1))
 (segment (start 195 136) (end 197 136) (width 0.2) (layer B.Cu) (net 1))
 (segment (start 211.36 137.46) (end 211.36 136) (width 0.2) (layer B.Cu) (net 1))
 (segment (start 211.36 136) (end 211.5 136) (width 0.2) (layer B.Cu) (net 1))
 (segment (start 211.5 136) (end 224 136) (width 0.2) (layer B.Cu) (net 1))
 (segment (start 224.06 137.46) (end 223.768 137.46) (width 0.2) (layer B.Cu) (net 1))
 (segment (start 224.06 137.46) (end 224.06 136) (width 0.2) (layer B.Cu) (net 1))
 (segment (start 224.06 136) (end 224 136) (width 0.2) (layer B.Cu) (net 1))
 (segment (start 229.14 136.14) (end 229.14 137.46) (width 0.2) (layer B.Cu) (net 1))
 (segment (start 238 140) (end 241.5 143) (width 0.2) (layer B.Cu) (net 1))
 (via (at 241.5 143) (size 0.9) (drill 0.6) (layers F.Cu B.Cu) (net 1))
 (segment (start 236.76 140) (end 238 140) (width 0.2) (layer B.Cu) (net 1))
 (segment (start 238 136) (end 229 136) (width 0.2) (layer B.Cu) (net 1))
 (segment (start 238 140) (end 238 136) (width 0.2) (layer B.Cu) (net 1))
 (segment (start 224 136) (end 229 136) (width 0.2) (layer B.Cu) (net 1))
 (segment (start 229 136) (end 229.14 136.14) (width 0.2) (layer B.Cu) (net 1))
 (segment (start 234.85 148.6) (end 234.85 150.8) (width 0.2) (layer F.Cu) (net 10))
 (segment (start 234.95 152.9) (end 234.95 150.9) (width 0.2) (layer F.Cu) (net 10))
 (segment (start 234.95 150.9) (end 234.85 150.8) (width 0.2) (layer F.Cu) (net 10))
 (segment (start 234.85 143.65) (end 234.85 146.4) (width 0.2) (layer F.Cu) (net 10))
 (segment (start 234.7 143.5) (end 234.85 143.65) (width 0.2) (layer F.Cu) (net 10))
 (segment (start 234.85 148.6) (end 234.85 146.4) (width 0.2) (layer F.Cu) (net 10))
 (segment (start 227.05 143.5) (end 234.7 143.5) (width 0.2) (layer F.Cu) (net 10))
 (segment (start 208.82 140) (end 212.32 143.5) (width 0.2) (layer F.Cu) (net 10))
 (segment (start 225.75 143.5) (end 212.32 143.5) (width 0.2) (layer F.Cu) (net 10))
 (segment (start 225.75 143.5) (end 227.05 143.5) (width 0.2) (layer F.Cu) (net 10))
 (segment (start 243.27 153.75) (end 242.05 153.75) (width 0.2) (layer F.Cu) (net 2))
 (segment (start 240 153.5) (end 237.55 151.05) (width 0.2) (layer F.Cu) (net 2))
 (via (at 240 153.5) (size 0.9) (drill 0.6) (layers F.Cu B.Cu) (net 2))
 (segment (start 241.7 153.5) (end 240 153.5) (width 0.2) (layer B.Cu) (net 2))
 (segment (start 242 153.8) (end 241.7 153.5) (width 0.2) (layer B.Cu) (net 2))
 (via (at 242 153.8) (size 0.9) (drill 0.6) (layers F.Cu B.Cu) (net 2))
 (segment (start 242.05 153.75) (end 242 153.8) (width 0.2) (layer F.Cu) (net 2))
 (segment (start 237.55 151.05) (end 237.55 150.8) (width 0.2) (layer F.Cu) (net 2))
 (segment (start 242.135 150.675) (end 242.135 152.615) (width 0.2) (layer F.Cu) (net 2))
 (segment (start 242.135 152.615) (end 243.27 153.75) (width 0.2) (layer F.Cu) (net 2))
 (segment (start 188.5 137.5) (end 188.5 137.46) (width 0.2) (layer B.Cu) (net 6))
 (segment (start 191.04 137.46) (end 188.5 137.46) (width 0.2) (layer B.Cu) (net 6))
 (segment (start 184.21 141.75) (end 188.5 137.46) (width 0.2) (layer F.Cu) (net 6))
 (segment (start 181.5 141.75) (end 184.21 141.75) (width 0.2) (layer F.Cu) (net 6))
 (segment (start 180.5 142.75) (end 181.5 141.75) (width 0.2) (layer F.Cu) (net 6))
 (segment (start 180.5 145.25) (end 180.5 142.75) (width 0.2) (layer F.Cu) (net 6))
 (segment (start 182.5 146.6) (end 182.5 145.25) (width 0.2) (layer F.Cu) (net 6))
 (segment (start 181.65 149.6) (end 180.5 149.6) (width 0.2) (layer F.Cu) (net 6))
 (segment (start 180.5 149.6) (end 180.5 145.25) (width 0.2) (layer F.Cu) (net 6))
 (segment (start 182.5 145.25) (end 180.5 145.25) (width 0.2) (layer F.Cu) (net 6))
 (segment (start 236.2 147.25) (end 237.55 148.6) (width 0.2) (layer F.Cu) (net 9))
 (segment (start 236.2 143.7) (end 236.2 147.25) (width 0.2) (layer F.Cu) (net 9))
 (segment (start 235.25 142.75) (end 236.2 143.7) (width 0.2) (layer F.Cu) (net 9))
 (segment (start 239.595 150.675) (end 239.595 150.645) (width 0.2) (layer F.Cu) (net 9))
 (segment (start 239.595 150.645) (end 237.55 148.6) (width 0.2) (layer F.Cu) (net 9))
 (segment (start 223 142.75) (end 235.25 142.75) (width 0.2) (layer F.Cu) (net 9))
 (segment (start 221.52 140) (end 221.52 141.27) (width 0.2) (layer F.Cu) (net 9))
 (segment (start 223 142.75) (end 221.52 141.27) (width 0.2) (layer F.Cu) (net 9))
 (segment (start 235.23 142) (end 223.75 142) (width 0.2) (layer F.Cu) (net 8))
 (segment (start 223.75 142) (end 222.75 141) (width 0.2) (layer F.Cu) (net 8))
 (segment (start 222.75 141) (end 222.75 138.69) (width 0.2) (layer F.Cu) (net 8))
 (segment (start 221.52 137.46) (end 222.75 138.69) (width 0.2) (layer F.Cu) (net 8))
 (segment (start 238 142) (end 235.23 142) (width 0.2) (layer F.Cu) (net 8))
 (segment (start 238.5 142.5) (end 238 142) (width 0.2) (layer F.Cu) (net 8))
 (segment (start 238.5 145) (end 238.5 142.5) (width 0.2) (layer F.Cu) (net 8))
 (segment (start 239 145.5) (end 238.45 145.5) (width 0.2) (layer F.Cu) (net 8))
 (segment (start 239 145.5) (end 238.5 145) (width 0.2) (layer F.Cu) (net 8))
 (segment (start 240.5 145.5) (end 239 145.5) (width 0.2) (layer F.Cu) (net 8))
 (segment (start 238.45 145.5) (end 237.55 146.4) (width 0.2) (layer F.Cu) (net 8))
 (segment (start 240.865 147.635) (end 240.865 145.865) (width 0.2) (layer F.Cu) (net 8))
 (segment (start 240.865 147.635) (end 240.865 150.675) (width 0.2) (layer F.Cu) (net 8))
 (segment (start 240.865 145.865) (end 240.5 145.5) (width 0.2) (layer F.Cu) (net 8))
 (segment (start 183.45 143.9) (end 185.15 143.9) (width 0.2) (layer F.Cu) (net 3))
 (segment (start 185.15 143.9) (end 185.25 143.8) (width 0.2) (layer F.Cu) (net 3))
 (segment (start 183.55 144) (end 183.45 143.9) (width 0.2) (layer F.Cu) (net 3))
 (segment (start 181.55 143.9) (end 182.5 143.9) (width 0.2) (layer F.Cu) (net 3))
 (segment (start 182.5 143.9) (end 183.45 143.9) (width 0.2) (layer F.Cu) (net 3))
 (segment (start 183.55 149.6) (end 183.55 148.95) (width 0.2) (layer F.Cu) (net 4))
 (segment (start 183.55 148.95) (end 184.3 148.2) (width 0.2) (layer F.Cu) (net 4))
 (segment (start 184.3 148.2) (end 185.25 147.25) (width 0.2) (layer F.Cu) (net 4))
 (via (at 184.3 148.2) (size 0.9) (drill 0.6) (layers F.Cu B.Cu) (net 4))
 (segment (start 181.6 148.2) (end 184.3 148.2) (width 0.2) (layer B.Cu) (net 4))
 (segment (start 181.55 146.6) (end 181.55 148.15) (width 0.2) (layer F.Cu) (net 4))
 (segment (start 185.25 147.25) (end 185.25 145.6) (width 0.2) (layer F.Cu) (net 4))
 (via (at 181.6 148.2) (size 0.9) (drill 0.6) (layers F.Cu B.Cu) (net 4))
 (segment (start 181.55 148.15) (end 181.6 148.2) (width 0.2) (layer F.Cu) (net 4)))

